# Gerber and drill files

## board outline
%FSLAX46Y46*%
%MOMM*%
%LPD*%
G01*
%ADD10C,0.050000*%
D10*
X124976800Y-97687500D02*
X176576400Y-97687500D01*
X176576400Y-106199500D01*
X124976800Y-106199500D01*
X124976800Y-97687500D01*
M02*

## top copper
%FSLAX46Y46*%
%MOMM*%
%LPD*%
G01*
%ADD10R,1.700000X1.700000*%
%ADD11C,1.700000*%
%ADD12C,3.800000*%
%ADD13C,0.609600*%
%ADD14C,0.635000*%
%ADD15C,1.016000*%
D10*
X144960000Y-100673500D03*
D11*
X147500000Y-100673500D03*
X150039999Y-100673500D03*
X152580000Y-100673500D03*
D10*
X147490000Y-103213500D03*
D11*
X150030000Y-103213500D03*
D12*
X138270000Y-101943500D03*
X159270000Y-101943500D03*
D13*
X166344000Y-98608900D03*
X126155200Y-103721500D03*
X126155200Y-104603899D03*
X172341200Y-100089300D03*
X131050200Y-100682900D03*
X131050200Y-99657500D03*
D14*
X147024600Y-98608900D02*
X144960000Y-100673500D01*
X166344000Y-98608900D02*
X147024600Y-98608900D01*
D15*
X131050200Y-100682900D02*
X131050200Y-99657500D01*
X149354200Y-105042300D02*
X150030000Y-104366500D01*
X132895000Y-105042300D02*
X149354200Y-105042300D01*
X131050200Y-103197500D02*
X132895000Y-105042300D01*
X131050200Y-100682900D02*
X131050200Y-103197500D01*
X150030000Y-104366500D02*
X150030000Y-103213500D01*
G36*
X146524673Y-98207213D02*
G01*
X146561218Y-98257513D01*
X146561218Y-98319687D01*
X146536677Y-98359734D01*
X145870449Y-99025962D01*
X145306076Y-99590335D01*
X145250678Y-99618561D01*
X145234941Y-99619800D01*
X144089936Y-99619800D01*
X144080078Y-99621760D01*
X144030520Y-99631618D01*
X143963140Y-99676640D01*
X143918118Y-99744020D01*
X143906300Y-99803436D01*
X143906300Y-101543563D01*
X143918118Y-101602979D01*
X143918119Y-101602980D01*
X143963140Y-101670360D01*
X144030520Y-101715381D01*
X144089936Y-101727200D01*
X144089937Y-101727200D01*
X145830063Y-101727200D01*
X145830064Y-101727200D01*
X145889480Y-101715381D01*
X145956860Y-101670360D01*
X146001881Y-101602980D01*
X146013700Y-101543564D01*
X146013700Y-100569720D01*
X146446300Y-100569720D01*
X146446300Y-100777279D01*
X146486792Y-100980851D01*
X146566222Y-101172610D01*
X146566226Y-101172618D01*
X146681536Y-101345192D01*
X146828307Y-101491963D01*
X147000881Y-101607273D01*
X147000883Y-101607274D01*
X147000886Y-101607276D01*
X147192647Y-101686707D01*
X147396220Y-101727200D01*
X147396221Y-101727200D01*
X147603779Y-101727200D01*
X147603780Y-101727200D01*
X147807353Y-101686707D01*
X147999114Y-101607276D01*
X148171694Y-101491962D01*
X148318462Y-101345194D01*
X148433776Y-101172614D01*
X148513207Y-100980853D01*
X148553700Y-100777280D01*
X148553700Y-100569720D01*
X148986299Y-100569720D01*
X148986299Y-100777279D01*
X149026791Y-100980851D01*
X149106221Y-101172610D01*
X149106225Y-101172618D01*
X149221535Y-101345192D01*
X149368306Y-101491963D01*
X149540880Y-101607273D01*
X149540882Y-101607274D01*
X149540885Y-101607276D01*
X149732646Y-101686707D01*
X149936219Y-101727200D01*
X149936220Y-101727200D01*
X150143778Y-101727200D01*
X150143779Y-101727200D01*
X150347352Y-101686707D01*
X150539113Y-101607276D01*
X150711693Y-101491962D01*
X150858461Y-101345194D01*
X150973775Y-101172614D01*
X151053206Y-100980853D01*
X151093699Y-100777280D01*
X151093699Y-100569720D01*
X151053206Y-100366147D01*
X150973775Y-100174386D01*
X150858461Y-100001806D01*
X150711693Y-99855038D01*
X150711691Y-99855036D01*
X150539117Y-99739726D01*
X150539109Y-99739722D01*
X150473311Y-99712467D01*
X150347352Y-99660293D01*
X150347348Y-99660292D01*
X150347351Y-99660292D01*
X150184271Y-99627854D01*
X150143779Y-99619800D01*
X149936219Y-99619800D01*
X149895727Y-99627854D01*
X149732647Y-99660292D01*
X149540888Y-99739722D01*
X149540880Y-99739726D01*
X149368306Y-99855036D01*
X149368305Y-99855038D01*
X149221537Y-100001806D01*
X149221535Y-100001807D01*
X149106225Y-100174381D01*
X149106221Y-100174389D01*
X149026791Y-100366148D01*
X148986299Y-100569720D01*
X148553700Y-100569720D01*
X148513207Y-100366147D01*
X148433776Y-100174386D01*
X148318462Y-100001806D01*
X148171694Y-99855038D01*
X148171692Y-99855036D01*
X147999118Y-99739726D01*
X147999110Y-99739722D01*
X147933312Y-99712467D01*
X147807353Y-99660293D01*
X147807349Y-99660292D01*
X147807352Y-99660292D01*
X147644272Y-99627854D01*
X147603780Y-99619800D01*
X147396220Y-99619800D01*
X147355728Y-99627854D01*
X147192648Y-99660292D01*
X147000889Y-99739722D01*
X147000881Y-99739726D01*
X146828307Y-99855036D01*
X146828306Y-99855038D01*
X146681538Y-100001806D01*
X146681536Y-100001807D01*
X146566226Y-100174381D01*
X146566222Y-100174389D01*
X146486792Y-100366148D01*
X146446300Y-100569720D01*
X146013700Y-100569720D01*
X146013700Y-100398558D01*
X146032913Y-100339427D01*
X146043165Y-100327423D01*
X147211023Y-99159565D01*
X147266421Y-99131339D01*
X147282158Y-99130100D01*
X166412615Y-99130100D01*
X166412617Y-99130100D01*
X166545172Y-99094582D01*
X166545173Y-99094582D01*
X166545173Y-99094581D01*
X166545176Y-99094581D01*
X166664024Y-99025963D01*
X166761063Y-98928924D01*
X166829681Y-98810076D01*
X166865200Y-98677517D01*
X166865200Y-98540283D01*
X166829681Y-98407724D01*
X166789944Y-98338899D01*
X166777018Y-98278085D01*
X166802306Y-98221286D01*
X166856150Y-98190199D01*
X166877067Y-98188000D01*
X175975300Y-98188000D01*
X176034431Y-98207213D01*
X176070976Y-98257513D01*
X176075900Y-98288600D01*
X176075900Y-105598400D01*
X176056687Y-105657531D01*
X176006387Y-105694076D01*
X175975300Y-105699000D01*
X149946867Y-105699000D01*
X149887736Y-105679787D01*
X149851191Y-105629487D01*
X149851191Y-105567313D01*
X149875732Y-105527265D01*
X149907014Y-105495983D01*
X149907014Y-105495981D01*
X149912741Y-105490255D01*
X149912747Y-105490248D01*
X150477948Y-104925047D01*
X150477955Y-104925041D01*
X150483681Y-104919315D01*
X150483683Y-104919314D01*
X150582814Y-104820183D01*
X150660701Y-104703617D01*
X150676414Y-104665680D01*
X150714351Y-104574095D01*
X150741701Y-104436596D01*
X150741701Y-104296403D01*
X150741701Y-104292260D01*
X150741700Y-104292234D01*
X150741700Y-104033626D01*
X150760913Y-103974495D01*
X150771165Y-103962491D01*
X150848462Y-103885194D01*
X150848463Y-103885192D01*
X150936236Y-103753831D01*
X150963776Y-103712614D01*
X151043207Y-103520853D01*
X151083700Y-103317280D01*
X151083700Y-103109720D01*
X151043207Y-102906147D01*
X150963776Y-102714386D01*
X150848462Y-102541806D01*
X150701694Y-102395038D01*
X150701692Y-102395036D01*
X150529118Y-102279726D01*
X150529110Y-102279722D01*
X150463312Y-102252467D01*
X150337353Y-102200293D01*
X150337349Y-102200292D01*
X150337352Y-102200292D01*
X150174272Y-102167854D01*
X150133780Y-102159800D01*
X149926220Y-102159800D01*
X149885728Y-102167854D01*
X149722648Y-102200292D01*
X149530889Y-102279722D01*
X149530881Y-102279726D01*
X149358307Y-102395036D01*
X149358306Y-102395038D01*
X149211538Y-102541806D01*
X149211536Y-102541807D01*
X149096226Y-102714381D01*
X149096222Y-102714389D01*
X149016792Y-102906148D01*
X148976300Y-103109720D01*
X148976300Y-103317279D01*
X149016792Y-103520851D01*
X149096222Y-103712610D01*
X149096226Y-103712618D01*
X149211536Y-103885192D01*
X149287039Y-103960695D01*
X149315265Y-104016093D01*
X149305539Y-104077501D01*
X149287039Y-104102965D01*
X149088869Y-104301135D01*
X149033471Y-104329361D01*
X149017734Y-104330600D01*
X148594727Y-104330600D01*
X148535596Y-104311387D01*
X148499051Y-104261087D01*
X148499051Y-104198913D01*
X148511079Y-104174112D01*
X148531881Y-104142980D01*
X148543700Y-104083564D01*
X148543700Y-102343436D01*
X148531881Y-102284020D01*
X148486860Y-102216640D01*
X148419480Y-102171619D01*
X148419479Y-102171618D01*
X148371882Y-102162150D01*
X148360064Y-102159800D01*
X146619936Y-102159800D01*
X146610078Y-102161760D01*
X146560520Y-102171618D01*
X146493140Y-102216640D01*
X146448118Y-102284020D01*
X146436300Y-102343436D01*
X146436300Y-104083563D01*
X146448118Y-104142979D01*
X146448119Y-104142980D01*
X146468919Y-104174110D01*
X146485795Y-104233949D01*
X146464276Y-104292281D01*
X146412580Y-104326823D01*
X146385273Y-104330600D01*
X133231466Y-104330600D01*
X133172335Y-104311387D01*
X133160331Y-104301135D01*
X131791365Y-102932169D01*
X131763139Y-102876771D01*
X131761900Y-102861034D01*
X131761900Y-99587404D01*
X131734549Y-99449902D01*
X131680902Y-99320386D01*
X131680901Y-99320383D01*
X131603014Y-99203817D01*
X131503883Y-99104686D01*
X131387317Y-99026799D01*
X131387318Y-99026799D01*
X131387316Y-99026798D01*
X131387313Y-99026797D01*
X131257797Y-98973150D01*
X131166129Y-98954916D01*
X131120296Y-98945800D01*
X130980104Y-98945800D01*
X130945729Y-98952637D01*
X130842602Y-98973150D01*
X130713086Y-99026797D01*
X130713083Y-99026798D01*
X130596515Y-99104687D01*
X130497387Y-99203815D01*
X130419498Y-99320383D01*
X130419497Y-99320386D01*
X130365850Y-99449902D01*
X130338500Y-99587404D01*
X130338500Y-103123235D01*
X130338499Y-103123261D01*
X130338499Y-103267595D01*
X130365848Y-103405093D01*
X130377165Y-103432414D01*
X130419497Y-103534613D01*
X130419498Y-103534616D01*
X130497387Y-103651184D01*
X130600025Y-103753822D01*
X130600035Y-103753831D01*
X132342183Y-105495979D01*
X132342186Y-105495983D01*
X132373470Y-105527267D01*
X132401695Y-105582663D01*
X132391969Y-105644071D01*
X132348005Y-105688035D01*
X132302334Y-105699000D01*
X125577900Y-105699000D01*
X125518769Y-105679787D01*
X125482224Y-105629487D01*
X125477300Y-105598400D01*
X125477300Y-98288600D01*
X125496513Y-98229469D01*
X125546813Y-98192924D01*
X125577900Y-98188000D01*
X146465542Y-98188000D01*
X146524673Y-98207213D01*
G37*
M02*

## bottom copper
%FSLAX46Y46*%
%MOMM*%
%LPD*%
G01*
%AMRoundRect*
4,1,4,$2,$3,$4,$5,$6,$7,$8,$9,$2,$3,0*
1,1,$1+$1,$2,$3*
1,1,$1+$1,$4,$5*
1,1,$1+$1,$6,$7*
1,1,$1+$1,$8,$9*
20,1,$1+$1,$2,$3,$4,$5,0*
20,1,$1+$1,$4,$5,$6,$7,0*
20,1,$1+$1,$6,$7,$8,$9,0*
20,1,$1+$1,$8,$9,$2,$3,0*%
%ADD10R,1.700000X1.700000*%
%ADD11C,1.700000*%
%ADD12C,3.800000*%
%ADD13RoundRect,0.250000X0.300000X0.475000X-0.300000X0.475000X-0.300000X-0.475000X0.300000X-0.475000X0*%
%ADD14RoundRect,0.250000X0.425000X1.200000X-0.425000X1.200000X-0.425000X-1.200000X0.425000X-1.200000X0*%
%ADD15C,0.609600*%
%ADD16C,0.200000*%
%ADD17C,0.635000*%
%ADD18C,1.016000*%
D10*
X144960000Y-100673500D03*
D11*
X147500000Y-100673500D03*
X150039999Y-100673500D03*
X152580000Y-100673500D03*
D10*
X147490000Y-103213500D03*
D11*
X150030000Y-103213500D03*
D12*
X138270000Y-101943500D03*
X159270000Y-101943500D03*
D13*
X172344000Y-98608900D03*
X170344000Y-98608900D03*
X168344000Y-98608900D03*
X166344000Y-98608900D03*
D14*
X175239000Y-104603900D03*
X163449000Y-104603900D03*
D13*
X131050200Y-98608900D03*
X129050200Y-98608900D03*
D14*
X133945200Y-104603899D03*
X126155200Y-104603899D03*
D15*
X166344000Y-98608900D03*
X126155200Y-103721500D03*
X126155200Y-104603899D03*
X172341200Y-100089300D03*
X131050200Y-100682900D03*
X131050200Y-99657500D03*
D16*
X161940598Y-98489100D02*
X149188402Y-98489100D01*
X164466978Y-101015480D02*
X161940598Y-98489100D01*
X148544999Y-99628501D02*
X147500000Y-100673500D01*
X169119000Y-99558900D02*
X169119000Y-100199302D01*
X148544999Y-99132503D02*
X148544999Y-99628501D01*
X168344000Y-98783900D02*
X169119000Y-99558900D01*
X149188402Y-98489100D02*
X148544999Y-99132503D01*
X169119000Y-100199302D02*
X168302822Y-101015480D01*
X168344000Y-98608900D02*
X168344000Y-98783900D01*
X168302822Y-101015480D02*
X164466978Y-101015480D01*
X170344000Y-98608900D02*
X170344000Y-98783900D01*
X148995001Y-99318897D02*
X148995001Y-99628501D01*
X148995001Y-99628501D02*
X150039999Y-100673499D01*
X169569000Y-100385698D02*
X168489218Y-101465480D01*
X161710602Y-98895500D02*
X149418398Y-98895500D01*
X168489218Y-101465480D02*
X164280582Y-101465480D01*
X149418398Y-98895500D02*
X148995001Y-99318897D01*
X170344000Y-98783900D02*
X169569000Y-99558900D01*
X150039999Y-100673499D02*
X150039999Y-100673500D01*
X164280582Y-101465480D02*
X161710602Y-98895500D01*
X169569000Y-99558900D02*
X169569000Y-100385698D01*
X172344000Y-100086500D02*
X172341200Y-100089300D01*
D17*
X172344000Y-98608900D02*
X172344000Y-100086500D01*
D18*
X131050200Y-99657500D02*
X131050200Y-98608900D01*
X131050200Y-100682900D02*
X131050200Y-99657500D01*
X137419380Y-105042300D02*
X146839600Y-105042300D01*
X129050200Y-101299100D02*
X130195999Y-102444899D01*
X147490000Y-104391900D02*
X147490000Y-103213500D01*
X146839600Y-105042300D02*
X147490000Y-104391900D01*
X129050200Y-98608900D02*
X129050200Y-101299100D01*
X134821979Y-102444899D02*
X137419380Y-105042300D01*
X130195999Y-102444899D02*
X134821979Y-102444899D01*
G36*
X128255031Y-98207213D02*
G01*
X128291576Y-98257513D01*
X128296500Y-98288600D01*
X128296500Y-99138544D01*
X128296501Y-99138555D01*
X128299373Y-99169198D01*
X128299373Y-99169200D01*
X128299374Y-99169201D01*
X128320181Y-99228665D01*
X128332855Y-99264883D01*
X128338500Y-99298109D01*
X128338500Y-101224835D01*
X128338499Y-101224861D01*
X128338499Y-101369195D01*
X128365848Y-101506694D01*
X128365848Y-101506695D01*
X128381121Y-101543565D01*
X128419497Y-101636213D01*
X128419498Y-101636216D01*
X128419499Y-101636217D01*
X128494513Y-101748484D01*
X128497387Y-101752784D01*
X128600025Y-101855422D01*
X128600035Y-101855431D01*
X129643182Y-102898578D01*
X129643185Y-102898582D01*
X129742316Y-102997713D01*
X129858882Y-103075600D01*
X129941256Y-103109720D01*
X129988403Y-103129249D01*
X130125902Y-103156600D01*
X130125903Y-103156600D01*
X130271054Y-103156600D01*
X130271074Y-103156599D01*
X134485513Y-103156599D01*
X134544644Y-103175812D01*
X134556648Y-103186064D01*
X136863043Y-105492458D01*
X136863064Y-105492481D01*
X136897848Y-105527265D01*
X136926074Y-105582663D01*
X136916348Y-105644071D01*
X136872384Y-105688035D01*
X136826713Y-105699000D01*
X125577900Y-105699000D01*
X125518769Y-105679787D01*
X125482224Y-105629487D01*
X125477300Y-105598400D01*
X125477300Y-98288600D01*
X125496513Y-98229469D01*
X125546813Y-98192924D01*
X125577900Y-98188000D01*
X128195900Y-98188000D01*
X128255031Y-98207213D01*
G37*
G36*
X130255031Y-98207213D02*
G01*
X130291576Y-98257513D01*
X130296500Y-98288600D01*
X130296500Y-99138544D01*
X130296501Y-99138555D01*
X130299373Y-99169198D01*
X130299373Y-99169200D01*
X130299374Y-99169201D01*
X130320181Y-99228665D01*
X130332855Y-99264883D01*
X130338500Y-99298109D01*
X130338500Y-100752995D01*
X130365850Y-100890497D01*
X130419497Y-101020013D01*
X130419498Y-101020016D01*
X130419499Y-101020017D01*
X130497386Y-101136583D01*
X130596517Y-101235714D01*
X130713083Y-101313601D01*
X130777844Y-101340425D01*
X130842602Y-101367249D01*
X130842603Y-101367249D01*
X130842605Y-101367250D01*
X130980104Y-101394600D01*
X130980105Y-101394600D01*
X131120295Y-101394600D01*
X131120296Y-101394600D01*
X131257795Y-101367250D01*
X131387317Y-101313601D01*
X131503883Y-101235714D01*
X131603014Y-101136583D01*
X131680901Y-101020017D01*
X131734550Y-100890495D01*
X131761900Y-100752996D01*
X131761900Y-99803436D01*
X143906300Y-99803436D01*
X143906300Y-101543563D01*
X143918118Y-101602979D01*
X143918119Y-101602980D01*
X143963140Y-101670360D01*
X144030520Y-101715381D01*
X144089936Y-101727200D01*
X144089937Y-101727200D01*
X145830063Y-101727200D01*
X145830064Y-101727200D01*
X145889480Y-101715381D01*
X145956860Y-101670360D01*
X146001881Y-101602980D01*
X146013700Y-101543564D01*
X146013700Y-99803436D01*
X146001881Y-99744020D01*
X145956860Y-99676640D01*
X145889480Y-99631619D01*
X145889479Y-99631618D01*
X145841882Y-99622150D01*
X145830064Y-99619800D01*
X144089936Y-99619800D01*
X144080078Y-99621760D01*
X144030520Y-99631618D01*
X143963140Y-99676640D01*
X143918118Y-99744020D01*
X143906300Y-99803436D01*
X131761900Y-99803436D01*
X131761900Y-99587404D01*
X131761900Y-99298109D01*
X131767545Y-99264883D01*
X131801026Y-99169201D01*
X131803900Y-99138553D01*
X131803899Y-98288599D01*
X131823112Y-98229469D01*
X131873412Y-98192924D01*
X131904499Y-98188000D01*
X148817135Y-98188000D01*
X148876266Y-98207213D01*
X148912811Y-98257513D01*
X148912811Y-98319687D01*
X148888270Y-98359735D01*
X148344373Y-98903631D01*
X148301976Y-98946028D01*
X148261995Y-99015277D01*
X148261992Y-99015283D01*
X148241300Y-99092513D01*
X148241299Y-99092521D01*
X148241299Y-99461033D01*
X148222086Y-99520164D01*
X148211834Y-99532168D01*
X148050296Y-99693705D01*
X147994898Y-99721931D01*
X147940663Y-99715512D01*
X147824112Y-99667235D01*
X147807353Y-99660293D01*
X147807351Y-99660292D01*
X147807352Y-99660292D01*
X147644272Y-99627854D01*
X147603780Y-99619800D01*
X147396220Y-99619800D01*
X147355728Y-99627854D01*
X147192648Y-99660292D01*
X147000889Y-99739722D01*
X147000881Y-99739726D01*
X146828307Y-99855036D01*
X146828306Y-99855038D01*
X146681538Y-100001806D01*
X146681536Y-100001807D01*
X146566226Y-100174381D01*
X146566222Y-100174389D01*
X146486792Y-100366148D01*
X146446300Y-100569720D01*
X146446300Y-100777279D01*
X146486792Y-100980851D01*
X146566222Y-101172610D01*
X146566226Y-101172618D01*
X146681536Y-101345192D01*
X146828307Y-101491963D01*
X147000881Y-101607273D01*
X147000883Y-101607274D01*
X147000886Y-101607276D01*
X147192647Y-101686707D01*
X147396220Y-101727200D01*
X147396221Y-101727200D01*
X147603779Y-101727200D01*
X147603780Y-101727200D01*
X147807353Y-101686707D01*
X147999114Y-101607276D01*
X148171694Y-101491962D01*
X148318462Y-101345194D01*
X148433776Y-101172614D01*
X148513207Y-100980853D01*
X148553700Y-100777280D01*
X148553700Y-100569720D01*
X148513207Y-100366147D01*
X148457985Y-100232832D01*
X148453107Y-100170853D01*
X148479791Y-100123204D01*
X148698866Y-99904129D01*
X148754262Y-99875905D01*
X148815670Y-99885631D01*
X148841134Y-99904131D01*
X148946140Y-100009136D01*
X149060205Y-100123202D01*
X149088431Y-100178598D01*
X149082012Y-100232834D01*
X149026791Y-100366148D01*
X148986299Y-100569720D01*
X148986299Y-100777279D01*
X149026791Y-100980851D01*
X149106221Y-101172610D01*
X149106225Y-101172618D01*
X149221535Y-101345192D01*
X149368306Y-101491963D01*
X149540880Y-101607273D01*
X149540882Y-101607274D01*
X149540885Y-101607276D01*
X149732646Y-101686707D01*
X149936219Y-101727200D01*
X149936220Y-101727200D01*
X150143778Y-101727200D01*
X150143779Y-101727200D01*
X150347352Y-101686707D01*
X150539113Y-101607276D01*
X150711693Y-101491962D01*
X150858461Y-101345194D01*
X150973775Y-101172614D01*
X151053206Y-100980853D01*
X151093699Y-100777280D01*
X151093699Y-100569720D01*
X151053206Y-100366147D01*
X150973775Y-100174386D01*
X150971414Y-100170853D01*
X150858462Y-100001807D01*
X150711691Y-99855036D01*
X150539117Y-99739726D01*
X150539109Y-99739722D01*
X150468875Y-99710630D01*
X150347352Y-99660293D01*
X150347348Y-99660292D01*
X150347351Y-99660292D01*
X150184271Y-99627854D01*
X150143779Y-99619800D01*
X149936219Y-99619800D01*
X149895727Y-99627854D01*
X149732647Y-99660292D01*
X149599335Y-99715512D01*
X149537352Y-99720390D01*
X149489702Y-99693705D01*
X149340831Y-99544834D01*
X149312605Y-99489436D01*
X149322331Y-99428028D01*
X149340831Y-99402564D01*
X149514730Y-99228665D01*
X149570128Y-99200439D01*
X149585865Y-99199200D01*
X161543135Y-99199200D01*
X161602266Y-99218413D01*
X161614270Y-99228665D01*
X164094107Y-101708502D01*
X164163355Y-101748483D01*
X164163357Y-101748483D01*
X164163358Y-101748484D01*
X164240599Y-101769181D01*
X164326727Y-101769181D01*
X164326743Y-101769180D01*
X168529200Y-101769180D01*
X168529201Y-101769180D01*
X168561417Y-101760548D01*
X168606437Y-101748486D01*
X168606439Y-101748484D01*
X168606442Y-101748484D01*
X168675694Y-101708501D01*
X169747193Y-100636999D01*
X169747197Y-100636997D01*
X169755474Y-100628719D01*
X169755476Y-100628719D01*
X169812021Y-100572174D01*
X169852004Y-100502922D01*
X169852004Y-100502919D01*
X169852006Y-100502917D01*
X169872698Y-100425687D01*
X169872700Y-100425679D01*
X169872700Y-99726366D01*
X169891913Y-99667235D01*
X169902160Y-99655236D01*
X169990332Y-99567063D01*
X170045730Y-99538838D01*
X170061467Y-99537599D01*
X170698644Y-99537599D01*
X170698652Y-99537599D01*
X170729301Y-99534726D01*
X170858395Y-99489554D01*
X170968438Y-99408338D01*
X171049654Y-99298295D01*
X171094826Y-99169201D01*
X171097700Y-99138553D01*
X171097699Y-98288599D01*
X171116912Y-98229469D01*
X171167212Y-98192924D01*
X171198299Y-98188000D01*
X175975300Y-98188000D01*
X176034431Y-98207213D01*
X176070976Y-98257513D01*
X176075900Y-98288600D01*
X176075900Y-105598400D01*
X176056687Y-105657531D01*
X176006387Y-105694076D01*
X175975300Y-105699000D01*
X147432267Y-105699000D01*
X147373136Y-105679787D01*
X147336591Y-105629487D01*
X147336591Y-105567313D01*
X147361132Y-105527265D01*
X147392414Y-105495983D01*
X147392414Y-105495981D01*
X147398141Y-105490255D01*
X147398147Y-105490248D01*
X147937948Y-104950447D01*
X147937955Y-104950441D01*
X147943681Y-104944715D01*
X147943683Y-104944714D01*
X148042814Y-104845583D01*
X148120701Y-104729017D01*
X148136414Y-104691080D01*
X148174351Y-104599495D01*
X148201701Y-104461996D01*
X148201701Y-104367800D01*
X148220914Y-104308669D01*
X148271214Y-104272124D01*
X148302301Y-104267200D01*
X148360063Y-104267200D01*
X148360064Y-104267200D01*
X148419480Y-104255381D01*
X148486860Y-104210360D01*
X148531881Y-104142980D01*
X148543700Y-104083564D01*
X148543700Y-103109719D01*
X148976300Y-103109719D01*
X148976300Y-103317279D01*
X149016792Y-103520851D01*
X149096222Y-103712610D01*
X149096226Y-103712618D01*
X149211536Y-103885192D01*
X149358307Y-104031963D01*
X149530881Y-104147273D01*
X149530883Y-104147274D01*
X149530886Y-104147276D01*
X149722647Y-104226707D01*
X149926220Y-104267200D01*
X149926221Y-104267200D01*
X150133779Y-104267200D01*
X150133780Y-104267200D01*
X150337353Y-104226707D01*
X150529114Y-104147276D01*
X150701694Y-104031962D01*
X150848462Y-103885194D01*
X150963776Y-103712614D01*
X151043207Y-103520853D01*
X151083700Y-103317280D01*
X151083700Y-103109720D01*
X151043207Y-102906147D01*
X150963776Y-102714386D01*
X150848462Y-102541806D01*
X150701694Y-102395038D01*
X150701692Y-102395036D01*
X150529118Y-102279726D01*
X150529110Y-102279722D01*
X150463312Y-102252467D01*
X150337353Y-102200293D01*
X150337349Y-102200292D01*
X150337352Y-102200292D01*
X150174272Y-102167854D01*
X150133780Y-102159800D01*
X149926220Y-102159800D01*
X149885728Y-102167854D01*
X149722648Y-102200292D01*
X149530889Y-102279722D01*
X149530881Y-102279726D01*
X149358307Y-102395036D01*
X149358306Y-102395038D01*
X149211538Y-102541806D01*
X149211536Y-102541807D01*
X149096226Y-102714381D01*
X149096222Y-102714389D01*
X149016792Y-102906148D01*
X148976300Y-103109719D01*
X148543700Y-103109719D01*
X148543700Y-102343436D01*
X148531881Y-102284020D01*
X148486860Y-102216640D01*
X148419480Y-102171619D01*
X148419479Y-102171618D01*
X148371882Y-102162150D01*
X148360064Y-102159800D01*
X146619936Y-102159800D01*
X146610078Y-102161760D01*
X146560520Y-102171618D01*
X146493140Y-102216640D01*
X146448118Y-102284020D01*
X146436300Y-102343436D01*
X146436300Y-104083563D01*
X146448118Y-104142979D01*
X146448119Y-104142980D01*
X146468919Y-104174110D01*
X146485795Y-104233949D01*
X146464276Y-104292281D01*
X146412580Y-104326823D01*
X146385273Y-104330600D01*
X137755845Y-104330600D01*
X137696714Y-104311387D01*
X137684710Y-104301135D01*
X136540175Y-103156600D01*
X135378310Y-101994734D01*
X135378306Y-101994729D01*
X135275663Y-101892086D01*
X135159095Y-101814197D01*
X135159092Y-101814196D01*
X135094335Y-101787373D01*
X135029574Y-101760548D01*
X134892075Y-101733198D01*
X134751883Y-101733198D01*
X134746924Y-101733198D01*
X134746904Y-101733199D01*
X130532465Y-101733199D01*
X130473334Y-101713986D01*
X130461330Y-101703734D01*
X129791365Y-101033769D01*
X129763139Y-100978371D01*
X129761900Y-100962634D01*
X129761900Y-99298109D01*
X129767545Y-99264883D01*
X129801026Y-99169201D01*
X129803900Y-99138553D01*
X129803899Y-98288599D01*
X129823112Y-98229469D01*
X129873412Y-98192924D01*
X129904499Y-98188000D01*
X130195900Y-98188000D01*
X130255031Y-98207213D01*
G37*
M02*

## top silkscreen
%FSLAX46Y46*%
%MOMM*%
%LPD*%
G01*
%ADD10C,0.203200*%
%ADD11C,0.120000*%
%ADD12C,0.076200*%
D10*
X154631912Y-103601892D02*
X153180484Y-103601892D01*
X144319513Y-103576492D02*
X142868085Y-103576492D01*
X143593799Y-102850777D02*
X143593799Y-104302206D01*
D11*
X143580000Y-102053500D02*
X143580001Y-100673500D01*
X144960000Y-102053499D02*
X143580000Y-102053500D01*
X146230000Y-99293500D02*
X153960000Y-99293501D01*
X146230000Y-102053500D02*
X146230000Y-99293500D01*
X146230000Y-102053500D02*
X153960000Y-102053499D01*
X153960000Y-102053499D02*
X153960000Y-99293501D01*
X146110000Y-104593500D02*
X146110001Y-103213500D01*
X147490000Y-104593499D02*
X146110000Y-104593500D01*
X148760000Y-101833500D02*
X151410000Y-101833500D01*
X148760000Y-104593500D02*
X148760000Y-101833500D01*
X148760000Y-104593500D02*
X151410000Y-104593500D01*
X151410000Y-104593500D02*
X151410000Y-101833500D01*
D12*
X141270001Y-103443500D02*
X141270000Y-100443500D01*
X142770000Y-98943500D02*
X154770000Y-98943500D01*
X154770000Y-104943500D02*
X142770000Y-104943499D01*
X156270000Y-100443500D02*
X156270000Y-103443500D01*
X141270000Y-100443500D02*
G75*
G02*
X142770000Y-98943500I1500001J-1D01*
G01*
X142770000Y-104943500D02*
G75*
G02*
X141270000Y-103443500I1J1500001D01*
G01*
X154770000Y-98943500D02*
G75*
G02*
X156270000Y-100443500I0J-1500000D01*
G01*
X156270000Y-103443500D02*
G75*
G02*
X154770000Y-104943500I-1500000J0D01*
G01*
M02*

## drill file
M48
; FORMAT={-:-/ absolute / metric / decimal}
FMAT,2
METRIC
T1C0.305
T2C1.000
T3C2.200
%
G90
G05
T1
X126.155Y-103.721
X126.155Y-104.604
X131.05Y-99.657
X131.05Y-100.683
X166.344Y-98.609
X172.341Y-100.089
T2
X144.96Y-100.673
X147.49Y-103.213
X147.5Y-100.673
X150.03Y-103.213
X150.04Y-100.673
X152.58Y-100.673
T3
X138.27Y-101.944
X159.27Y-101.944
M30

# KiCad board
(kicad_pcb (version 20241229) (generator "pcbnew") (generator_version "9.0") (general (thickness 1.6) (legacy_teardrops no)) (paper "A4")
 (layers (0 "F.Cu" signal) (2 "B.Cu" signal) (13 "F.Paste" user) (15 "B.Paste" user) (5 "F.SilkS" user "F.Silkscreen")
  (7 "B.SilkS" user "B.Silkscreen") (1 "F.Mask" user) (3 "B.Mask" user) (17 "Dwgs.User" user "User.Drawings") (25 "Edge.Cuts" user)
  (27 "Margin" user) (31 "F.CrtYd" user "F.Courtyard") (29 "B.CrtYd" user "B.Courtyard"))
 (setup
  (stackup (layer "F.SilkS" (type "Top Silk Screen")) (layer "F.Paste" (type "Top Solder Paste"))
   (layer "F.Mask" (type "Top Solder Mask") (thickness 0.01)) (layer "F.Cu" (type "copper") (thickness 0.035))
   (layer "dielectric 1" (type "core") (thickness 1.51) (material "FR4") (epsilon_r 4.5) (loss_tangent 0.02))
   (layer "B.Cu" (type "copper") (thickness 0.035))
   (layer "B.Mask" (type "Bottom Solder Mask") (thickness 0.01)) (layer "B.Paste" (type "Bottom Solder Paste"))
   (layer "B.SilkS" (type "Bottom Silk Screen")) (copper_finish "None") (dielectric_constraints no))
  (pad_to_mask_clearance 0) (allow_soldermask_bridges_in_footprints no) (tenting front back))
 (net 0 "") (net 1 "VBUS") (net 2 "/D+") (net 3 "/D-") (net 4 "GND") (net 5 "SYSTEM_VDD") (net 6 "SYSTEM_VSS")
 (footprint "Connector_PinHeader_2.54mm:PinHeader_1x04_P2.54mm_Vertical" (layer "F.Cu") (at 144.96 100.6735 90)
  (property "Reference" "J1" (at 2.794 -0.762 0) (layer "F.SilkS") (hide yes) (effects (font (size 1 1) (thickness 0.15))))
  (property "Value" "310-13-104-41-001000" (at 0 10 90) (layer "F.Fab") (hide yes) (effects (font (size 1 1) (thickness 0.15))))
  (fp_line (start -1.38 -1.38) (end 0 -1.379999) (stroke (width 0.12) (type solid)) (layer "F.SilkS"))
  (fp_line (start -1.379999 0) (end -1.38 -1.38) (stroke (width 0.12) (type solid)) (layer "F.SilkS"))
  (fp_line (start 1.38 1.27) (end 1.379999 9) (stroke (width 0.12) (type solid)) (layer "F.SilkS"))
  (fp_line (start -1.38 1.27) (end 1.38 1.27) (stroke (width 0.12) (type solid)) (layer "F.SilkS"))
  (fp_line (start -1.38 1.27) (end -1.379999 9) (stroke (width 0.12) (type solid)) (layer "F.SilkS"))
  (fp_line (start -1.379999 9) (end 1.379999 9) (stroke (width 0.12) (type solid)) (layer "F.SilkS"))
  (pad "1" thru_hole rect (at 0 0 90) (size 1.7 1.7) (drill 1) (layers "*.Cu" "*.Mask") (remove_unused_layers no) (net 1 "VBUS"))
  (pad "2" thru_hole circle (at 0 2.54 90) (size 1.7 1.7) (drill 1) (layers "*.Cu" "*.Mask") (remove_unused_layers no) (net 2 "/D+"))
  (pad "3" thru_hole circle (at 0 5.079999 90) (size 1.7 1.7) (drill 1) (layers "*.Cu" "*.Mask") (remove_unused_layers no) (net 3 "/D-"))
  (pad "4" thru_hole circle (at 0 7.62 90) (size 1.7 1.7) (drill 1) (layers "*.Cu" "*.Mask") (remove_unused_layers no) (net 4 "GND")))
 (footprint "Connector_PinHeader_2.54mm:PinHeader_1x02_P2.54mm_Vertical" (layer "F.Cu") (at 147.49 103.2135 90)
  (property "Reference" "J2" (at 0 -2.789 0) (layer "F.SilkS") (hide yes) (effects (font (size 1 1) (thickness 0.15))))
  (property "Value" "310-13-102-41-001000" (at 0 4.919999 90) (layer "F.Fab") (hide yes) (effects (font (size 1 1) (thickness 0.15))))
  (fp_line (start -1.38 -1.38) (end 0 -1.379999) (stroke (width 0.12) (type solid)) (layer "F.SilkS"))
  (fp_line (start -1.379999 0) (end -1.38 -1.38) (stroke (width 0.12) (type solid)) (layer "F.SilkS"))
  (fp_line (start 1.38 1.27) (end 1.38 3.92) (stroke (width 0.12) (type solid)) (layer "F.SilkS"))
  (fp_line (start -1.38 1.27) (end 1.38 1.27) (stroke (width 0.12) (type solid)) (layer "F.SilkS"))
  (fp_line (start -1.38 1.27) (end -1.38 3.92) (stroke (width 0.12) (type solid)) (layer "F.SilkS"))
  (fp_line (start -1.38 3.92) (end 1.38 3.92) (stroke (width 0.12) (type solid)) (layer "F.SilkS"))
  (pad "1" thru_hole rect (at 0 0 90) (size 1.7 1.7) (drill 1) (layers "*.Cu" "*.Mask") (remove_unused_layers no) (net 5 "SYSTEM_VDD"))
  (pad "2" thru_hole circle (at 0 2.54 90) (size 1.7 1.7) (drill 1) (layers "*.Cu" "*.Mask") (remove_unused_layers no) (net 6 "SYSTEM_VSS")))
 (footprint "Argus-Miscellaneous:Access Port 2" (layer "F.Cu") (at 148.77 101.9435)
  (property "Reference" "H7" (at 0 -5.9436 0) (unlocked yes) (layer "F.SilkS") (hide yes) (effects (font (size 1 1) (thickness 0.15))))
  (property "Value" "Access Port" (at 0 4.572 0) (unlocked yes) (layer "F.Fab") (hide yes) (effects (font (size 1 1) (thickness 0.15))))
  (fp_line (start -7.499999 1.5) (end -7.5 -1.5) (stroke (width 0.0762) (type solid)) (layer "F.SilkS"))
  (fp_line (start -6 -3) (end 6 -3) (stroke (width 0.0762) (type solid)) (layer "F.SilkS"))
  (fp_line (start 6 3) (end -6 2.999999) (stroke (width 0.0762) (type solid)) (layer "F.SilkS"))
  (fp_line (start 7.5 -1.5) (end 7.5 1.5) (stroke (width 0.0762) (type solid)) (layer "F.SilkS"))
  (fp_arc (start -7.5 -1.5) (mid -7.06066 -2.56066) (end -6 -3) (stroke (width 0.0762) (type solid)) (layer "F.SilkS"))
  (fp_arc (start -6 3) (mid -7.06066 2.56066) (end -7.5 1.5) (stroke (width 0.0762) (type solid)) (layer "F.SilkS"))
  (fp_arc (start 6 -3) (mid 7.06066 -2.56066) (end 7.5 -1.5) (stroke (width 0.0762) (type solid)) (layer "F.SilkS"))
  (fp_arc (start 7.5 1.5) (mid 7.06066 2.56066) (end 6 3) (stroke (width 0.0762) (type solid)) (layer "F.SilkS"))
  (pad "1" thru_hole circle (at -10.5 0) (size 3.8 3.8) (drill 2.2) (layers "*.Cu" "*.Mask") (remove_unused_layers no) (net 4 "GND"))
  (pad "1" thru_hole circle (at 10.5 0) (size 3.8 3.8) (drill 2.2) (layers "*.Cu" "*.Mask") (remove_unused_layers no) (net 4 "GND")))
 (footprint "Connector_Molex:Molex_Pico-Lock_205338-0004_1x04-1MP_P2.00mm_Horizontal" (layer "B.Cu") (at 169.344 101.9689 180)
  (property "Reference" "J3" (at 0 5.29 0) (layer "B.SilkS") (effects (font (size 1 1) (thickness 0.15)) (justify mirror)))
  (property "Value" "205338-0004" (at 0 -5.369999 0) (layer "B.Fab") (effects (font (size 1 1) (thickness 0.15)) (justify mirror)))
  (pad "1" smd roundrect (at -3 3.36 180) (size 1.1 1.45) (layers "B.Cu" "B.Mask" "B.Paste") (roundrect_rratio 0.227273) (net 4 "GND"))
  (pad "2" smd roundrect (at -1 3.36 180) (size 1.1 1.45) (layers "B.Cu" "B.Mask" "B.Paste") (roundrect_rratio 0.227273) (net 3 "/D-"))
  (pad "3" smd roundrect (at 1 3.36 180) (size 1.1 1.45) (layers "B.Cu" "B.Mask" "B.Paste") (roundrect_rratio 0.227273) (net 2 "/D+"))
  (pad "4" smd roundrect (at 3 3.36 180) (size 1.1 1.45) (layers "B.Cu" "B.Mask" "B.Paste") (roundrect_rratio 0.227273) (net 1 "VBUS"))
  (pad "MP" smd roundrect (at -5.895 -2.635 180) (size 1.35 2.9) (layers "B.Cu" "B.Mask" "B.Paste") (roundrect_rratio 0.185185)
   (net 4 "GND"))
  (pad "MP" smd roundrect (at 5.895 -2.635 180) (size 1.35 2.9) (layers "B.Cu" "B.Mask" "B.Paste") (roundrect_rratio 0.185185) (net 4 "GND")))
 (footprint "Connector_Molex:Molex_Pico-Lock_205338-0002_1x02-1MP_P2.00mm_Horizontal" (layer "B.Cu") (at 130.0502 101.9689 180)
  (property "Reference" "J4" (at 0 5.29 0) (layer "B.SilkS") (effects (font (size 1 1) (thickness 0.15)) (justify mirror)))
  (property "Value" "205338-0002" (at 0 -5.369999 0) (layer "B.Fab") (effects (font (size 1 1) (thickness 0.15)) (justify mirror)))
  (pad "1" smd roundrect (at -1 3.36 180) (size 1.1 1.45) (layers "B.Cu" "B.Mask" "B.Paste") (roundrect_rratio 0.227273)
   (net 6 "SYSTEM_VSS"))
  (pad "2" smd roundrect (at 1 3.36 180) (size 1.1 1.45) (layers "B.Cu" "B.Mask" "B.Paste") (roundrect_rratio 0.227273) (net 5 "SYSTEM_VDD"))
  (pad "MP" smd roundrect (at -3.895 -2.634999 180) (size 1.35 2.9) (layers "B.Cu" "B.Mask" "B.Paste") (roundrect_rratio 0.185185)
   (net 4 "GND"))
  (pad "MP" smd roundrect (at 3.895 -2.634999 180) (size 1.35 2.9) (layers "B.Cu" "B.Mask" "B.Paste") (roundrect_rratio 0.185185)
   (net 4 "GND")))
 (gr_rect (start 124.9768 97.6875) (end 176.5764 106.1995) (stroke (width 0.05) (type solid)) (fill no) (layer "Edge.Cuts"))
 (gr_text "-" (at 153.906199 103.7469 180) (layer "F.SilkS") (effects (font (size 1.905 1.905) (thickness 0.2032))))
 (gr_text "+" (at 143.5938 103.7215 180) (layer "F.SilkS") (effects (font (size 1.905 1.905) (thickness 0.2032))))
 (segment (start 161.940598 98.4891) (end 149.188402 98.4891) (width 0.2) (layer "B.Cu") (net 2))
 (segment (start 164.466978 101.01548) (end 161.940598 98.4891) (width 0.2) (layer "B.Cu") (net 2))
 (segment (start 148.544999 99.628501) (end 147.5 100.6735) (width 0.2) (layer "B.Cu") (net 2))
 (segment (start 169.119 99.5589) (end 169.119 100.199302) (width 0.2) (layer "B.Cu") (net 2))
 (segment (start 148.544999 99.132503) (end 148.544999 99.628501) (width 0.2) (layer "B.Cu") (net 2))
 (segment (start 168.344 98.7839) (end 169.119 99.5589) (width 0.2) (layer "B.Cu") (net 2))
 (segment (start 149.188402 98.4891) (end 148.544999 99.132503) (width 0.2) (layer "B.Cu") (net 2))
 (segment (start 169.119 100.199302) (end 168.302822 101.01548) (width 0.2) (layer "B.Cu") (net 2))
 (segment (start 168.344 98.6089) (end 168.344 98.7839) (width 0.2) (layer "B.Cu") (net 2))
 (segment (start 168.302822 101.01548) (end 164.466978 101.01548) (width 0.2) (layer "B.Cu") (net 2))
 (segment (start 147.0246 98.6089) (end 144.96 100.6735) (width 0.635) (layer "F.Cu") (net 1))
 (segment (start 166.344 98.6089) (end 147.0246 98.6089) (width 0.635) (layer "F.Cu") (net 1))
 (via (at 166.344 98.6089) (size 0.6096) (drill 0.3048) (layers "F.Cu" "B.Cu") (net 1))
 (segment (start 170.344 98.6089) (end 170.344 98.7839) (width 0.2) (layer "B.Cu") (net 3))
 (segment (start 148.995001 99.318897) (end 148.995001 99.628501) (width 0.2) (layer "B.Cu") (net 3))
 (segment (start 148.995001 99.628501) (end 150.039999 100.673499) (width 0.2) (layer "B.Cu") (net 3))
 (segment (start 169.569 100.385698) (end 168.489218 101.46548) (width 0.2) (layer "B.Cu") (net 3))
 (segment (start 161.710602 98.8955) (end 149.418398 98.8955) (width 0.2) (layer "B.Cu") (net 3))
 (segment (start 168.489218 101.46548) (end 164.280582 101.46548) (width 0.2) (layer "B.Cu") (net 3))
 (segment (start 149.418398 98.8955) (end 148.995001 99.318897) (width 0.2) (layer "B.Cu") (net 3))
 (segment (start 170.344 98.7839) (end 169.569 99.5589) (width 0.2) (layer "B.Cu") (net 3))
 (segment (start 150.039999 100.673499) (end 150.039999 100.6735) (width 0.2) (layer "B.Cu") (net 3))
 (segment (start 164.280582 101.46548) (end 161.710602 98.8955) (width 0.2) (layer "B.Cu") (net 3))
 (segment (start 169.569 99.5589) (end 169.569 100.385698) (width 0.2) (layer "B.Cu") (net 3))
 (via (at 126.1552 103.7215) (size 0.6096) (drill 0.3048) (layers "F.Cu" "B.Cu") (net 4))
 (via (at 126.1552 104.603899) (size 0.6096) (drill 0.3048) (layers "F.Cu" "B.Cu") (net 4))
 (via (at 172.3412 100.0893) (size 0.6096) (drill 0.3048) (layers "F.Cu" "B.Cu") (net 4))
 (segment (start 172.344 100.0865) (end 172.3412 100.0893) (width 0.2) (layer "B.Cu") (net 4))
 (segment (start 172.344 98.6089) (end 172.344 100.0865) (width 0.635) (layer "B.Cu") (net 4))
 (segment (start 131.0502 100.6829) (end 131.0502 99.6575) (width 1.016) (layer "F.Cu") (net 6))
 (segment (start 149.3542 105.0423) (end 150.03 104.3665) (width 1.016) (layer "F.Cu") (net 6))
 (segment (start 132.895 105.0423) (end 149.3542 105.0423) (width 1.016) (layer "F.Cu") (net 6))
 (segment (start 131.0502 103.1975) (end 132.895 105.0423) (width 1.016) (layer "F.Cu") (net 6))
 (segment (start 131.0502 100.6829) (end 131.0502 103.1975) (width 1.016) (layer "F.Cu") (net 6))
 (segment (start 150.03 104.3665) (end 150.03 103.2135) (width 1.016) (layer "F.Cu") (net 6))
 (via (at 131.0502 100.6829) (size 0.6096) (drill 0.3048) (layers "F.Cu" "B.Cu") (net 6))
 (via (at 131.0502 99.6575) (size 0.6096) (drill 0.3048) (layers "F.Cu" "B.Cu") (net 6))
 (segment (start 131.0502 99.6575) (end 131.0502 98.6089) (width 1.016) (layer "B.Cu") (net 6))
 (segment (start 131.0502 100.6829) (end 131.0502 99.6575) (width 1.016) (layer "B.Cu") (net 6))
 (segment (start 137.41938 105.0423) (end 146.8396 105.0423) (width 1.016) (layer "B.Cu") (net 5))
 (segment (start 129.0502 101.2991) (end 130.195999 102.444899) (width 1.016) (layer "B.Cu") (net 5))
 (segment (start 147.49 104.3919) (end 147.49 103.2135) (width 1.016) (layer "B.Cu") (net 5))
 (segment (start 146.8396 105.0423) (end 147.49 104.3919) (width 1.016) (layer "B.Cu") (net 5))
 (segment (start 129.0502 98.6089) (end 129.0502 101.2991) (width 1.016) (layer "B.Cu") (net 5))
 (segment (start 134.821979 102.444899) (end 137.41938 105.0423) (width 1.016) (layer "B.Cu") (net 5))
 (segment (start 130.195999 102.444899) (end 134.821979 102.444899) (width 1.016) (layer "B.Cu") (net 5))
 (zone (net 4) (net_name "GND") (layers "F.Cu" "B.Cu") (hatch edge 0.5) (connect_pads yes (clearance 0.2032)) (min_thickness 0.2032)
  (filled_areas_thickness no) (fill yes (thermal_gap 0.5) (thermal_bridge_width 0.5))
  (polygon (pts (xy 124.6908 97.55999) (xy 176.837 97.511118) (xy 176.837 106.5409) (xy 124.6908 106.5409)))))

